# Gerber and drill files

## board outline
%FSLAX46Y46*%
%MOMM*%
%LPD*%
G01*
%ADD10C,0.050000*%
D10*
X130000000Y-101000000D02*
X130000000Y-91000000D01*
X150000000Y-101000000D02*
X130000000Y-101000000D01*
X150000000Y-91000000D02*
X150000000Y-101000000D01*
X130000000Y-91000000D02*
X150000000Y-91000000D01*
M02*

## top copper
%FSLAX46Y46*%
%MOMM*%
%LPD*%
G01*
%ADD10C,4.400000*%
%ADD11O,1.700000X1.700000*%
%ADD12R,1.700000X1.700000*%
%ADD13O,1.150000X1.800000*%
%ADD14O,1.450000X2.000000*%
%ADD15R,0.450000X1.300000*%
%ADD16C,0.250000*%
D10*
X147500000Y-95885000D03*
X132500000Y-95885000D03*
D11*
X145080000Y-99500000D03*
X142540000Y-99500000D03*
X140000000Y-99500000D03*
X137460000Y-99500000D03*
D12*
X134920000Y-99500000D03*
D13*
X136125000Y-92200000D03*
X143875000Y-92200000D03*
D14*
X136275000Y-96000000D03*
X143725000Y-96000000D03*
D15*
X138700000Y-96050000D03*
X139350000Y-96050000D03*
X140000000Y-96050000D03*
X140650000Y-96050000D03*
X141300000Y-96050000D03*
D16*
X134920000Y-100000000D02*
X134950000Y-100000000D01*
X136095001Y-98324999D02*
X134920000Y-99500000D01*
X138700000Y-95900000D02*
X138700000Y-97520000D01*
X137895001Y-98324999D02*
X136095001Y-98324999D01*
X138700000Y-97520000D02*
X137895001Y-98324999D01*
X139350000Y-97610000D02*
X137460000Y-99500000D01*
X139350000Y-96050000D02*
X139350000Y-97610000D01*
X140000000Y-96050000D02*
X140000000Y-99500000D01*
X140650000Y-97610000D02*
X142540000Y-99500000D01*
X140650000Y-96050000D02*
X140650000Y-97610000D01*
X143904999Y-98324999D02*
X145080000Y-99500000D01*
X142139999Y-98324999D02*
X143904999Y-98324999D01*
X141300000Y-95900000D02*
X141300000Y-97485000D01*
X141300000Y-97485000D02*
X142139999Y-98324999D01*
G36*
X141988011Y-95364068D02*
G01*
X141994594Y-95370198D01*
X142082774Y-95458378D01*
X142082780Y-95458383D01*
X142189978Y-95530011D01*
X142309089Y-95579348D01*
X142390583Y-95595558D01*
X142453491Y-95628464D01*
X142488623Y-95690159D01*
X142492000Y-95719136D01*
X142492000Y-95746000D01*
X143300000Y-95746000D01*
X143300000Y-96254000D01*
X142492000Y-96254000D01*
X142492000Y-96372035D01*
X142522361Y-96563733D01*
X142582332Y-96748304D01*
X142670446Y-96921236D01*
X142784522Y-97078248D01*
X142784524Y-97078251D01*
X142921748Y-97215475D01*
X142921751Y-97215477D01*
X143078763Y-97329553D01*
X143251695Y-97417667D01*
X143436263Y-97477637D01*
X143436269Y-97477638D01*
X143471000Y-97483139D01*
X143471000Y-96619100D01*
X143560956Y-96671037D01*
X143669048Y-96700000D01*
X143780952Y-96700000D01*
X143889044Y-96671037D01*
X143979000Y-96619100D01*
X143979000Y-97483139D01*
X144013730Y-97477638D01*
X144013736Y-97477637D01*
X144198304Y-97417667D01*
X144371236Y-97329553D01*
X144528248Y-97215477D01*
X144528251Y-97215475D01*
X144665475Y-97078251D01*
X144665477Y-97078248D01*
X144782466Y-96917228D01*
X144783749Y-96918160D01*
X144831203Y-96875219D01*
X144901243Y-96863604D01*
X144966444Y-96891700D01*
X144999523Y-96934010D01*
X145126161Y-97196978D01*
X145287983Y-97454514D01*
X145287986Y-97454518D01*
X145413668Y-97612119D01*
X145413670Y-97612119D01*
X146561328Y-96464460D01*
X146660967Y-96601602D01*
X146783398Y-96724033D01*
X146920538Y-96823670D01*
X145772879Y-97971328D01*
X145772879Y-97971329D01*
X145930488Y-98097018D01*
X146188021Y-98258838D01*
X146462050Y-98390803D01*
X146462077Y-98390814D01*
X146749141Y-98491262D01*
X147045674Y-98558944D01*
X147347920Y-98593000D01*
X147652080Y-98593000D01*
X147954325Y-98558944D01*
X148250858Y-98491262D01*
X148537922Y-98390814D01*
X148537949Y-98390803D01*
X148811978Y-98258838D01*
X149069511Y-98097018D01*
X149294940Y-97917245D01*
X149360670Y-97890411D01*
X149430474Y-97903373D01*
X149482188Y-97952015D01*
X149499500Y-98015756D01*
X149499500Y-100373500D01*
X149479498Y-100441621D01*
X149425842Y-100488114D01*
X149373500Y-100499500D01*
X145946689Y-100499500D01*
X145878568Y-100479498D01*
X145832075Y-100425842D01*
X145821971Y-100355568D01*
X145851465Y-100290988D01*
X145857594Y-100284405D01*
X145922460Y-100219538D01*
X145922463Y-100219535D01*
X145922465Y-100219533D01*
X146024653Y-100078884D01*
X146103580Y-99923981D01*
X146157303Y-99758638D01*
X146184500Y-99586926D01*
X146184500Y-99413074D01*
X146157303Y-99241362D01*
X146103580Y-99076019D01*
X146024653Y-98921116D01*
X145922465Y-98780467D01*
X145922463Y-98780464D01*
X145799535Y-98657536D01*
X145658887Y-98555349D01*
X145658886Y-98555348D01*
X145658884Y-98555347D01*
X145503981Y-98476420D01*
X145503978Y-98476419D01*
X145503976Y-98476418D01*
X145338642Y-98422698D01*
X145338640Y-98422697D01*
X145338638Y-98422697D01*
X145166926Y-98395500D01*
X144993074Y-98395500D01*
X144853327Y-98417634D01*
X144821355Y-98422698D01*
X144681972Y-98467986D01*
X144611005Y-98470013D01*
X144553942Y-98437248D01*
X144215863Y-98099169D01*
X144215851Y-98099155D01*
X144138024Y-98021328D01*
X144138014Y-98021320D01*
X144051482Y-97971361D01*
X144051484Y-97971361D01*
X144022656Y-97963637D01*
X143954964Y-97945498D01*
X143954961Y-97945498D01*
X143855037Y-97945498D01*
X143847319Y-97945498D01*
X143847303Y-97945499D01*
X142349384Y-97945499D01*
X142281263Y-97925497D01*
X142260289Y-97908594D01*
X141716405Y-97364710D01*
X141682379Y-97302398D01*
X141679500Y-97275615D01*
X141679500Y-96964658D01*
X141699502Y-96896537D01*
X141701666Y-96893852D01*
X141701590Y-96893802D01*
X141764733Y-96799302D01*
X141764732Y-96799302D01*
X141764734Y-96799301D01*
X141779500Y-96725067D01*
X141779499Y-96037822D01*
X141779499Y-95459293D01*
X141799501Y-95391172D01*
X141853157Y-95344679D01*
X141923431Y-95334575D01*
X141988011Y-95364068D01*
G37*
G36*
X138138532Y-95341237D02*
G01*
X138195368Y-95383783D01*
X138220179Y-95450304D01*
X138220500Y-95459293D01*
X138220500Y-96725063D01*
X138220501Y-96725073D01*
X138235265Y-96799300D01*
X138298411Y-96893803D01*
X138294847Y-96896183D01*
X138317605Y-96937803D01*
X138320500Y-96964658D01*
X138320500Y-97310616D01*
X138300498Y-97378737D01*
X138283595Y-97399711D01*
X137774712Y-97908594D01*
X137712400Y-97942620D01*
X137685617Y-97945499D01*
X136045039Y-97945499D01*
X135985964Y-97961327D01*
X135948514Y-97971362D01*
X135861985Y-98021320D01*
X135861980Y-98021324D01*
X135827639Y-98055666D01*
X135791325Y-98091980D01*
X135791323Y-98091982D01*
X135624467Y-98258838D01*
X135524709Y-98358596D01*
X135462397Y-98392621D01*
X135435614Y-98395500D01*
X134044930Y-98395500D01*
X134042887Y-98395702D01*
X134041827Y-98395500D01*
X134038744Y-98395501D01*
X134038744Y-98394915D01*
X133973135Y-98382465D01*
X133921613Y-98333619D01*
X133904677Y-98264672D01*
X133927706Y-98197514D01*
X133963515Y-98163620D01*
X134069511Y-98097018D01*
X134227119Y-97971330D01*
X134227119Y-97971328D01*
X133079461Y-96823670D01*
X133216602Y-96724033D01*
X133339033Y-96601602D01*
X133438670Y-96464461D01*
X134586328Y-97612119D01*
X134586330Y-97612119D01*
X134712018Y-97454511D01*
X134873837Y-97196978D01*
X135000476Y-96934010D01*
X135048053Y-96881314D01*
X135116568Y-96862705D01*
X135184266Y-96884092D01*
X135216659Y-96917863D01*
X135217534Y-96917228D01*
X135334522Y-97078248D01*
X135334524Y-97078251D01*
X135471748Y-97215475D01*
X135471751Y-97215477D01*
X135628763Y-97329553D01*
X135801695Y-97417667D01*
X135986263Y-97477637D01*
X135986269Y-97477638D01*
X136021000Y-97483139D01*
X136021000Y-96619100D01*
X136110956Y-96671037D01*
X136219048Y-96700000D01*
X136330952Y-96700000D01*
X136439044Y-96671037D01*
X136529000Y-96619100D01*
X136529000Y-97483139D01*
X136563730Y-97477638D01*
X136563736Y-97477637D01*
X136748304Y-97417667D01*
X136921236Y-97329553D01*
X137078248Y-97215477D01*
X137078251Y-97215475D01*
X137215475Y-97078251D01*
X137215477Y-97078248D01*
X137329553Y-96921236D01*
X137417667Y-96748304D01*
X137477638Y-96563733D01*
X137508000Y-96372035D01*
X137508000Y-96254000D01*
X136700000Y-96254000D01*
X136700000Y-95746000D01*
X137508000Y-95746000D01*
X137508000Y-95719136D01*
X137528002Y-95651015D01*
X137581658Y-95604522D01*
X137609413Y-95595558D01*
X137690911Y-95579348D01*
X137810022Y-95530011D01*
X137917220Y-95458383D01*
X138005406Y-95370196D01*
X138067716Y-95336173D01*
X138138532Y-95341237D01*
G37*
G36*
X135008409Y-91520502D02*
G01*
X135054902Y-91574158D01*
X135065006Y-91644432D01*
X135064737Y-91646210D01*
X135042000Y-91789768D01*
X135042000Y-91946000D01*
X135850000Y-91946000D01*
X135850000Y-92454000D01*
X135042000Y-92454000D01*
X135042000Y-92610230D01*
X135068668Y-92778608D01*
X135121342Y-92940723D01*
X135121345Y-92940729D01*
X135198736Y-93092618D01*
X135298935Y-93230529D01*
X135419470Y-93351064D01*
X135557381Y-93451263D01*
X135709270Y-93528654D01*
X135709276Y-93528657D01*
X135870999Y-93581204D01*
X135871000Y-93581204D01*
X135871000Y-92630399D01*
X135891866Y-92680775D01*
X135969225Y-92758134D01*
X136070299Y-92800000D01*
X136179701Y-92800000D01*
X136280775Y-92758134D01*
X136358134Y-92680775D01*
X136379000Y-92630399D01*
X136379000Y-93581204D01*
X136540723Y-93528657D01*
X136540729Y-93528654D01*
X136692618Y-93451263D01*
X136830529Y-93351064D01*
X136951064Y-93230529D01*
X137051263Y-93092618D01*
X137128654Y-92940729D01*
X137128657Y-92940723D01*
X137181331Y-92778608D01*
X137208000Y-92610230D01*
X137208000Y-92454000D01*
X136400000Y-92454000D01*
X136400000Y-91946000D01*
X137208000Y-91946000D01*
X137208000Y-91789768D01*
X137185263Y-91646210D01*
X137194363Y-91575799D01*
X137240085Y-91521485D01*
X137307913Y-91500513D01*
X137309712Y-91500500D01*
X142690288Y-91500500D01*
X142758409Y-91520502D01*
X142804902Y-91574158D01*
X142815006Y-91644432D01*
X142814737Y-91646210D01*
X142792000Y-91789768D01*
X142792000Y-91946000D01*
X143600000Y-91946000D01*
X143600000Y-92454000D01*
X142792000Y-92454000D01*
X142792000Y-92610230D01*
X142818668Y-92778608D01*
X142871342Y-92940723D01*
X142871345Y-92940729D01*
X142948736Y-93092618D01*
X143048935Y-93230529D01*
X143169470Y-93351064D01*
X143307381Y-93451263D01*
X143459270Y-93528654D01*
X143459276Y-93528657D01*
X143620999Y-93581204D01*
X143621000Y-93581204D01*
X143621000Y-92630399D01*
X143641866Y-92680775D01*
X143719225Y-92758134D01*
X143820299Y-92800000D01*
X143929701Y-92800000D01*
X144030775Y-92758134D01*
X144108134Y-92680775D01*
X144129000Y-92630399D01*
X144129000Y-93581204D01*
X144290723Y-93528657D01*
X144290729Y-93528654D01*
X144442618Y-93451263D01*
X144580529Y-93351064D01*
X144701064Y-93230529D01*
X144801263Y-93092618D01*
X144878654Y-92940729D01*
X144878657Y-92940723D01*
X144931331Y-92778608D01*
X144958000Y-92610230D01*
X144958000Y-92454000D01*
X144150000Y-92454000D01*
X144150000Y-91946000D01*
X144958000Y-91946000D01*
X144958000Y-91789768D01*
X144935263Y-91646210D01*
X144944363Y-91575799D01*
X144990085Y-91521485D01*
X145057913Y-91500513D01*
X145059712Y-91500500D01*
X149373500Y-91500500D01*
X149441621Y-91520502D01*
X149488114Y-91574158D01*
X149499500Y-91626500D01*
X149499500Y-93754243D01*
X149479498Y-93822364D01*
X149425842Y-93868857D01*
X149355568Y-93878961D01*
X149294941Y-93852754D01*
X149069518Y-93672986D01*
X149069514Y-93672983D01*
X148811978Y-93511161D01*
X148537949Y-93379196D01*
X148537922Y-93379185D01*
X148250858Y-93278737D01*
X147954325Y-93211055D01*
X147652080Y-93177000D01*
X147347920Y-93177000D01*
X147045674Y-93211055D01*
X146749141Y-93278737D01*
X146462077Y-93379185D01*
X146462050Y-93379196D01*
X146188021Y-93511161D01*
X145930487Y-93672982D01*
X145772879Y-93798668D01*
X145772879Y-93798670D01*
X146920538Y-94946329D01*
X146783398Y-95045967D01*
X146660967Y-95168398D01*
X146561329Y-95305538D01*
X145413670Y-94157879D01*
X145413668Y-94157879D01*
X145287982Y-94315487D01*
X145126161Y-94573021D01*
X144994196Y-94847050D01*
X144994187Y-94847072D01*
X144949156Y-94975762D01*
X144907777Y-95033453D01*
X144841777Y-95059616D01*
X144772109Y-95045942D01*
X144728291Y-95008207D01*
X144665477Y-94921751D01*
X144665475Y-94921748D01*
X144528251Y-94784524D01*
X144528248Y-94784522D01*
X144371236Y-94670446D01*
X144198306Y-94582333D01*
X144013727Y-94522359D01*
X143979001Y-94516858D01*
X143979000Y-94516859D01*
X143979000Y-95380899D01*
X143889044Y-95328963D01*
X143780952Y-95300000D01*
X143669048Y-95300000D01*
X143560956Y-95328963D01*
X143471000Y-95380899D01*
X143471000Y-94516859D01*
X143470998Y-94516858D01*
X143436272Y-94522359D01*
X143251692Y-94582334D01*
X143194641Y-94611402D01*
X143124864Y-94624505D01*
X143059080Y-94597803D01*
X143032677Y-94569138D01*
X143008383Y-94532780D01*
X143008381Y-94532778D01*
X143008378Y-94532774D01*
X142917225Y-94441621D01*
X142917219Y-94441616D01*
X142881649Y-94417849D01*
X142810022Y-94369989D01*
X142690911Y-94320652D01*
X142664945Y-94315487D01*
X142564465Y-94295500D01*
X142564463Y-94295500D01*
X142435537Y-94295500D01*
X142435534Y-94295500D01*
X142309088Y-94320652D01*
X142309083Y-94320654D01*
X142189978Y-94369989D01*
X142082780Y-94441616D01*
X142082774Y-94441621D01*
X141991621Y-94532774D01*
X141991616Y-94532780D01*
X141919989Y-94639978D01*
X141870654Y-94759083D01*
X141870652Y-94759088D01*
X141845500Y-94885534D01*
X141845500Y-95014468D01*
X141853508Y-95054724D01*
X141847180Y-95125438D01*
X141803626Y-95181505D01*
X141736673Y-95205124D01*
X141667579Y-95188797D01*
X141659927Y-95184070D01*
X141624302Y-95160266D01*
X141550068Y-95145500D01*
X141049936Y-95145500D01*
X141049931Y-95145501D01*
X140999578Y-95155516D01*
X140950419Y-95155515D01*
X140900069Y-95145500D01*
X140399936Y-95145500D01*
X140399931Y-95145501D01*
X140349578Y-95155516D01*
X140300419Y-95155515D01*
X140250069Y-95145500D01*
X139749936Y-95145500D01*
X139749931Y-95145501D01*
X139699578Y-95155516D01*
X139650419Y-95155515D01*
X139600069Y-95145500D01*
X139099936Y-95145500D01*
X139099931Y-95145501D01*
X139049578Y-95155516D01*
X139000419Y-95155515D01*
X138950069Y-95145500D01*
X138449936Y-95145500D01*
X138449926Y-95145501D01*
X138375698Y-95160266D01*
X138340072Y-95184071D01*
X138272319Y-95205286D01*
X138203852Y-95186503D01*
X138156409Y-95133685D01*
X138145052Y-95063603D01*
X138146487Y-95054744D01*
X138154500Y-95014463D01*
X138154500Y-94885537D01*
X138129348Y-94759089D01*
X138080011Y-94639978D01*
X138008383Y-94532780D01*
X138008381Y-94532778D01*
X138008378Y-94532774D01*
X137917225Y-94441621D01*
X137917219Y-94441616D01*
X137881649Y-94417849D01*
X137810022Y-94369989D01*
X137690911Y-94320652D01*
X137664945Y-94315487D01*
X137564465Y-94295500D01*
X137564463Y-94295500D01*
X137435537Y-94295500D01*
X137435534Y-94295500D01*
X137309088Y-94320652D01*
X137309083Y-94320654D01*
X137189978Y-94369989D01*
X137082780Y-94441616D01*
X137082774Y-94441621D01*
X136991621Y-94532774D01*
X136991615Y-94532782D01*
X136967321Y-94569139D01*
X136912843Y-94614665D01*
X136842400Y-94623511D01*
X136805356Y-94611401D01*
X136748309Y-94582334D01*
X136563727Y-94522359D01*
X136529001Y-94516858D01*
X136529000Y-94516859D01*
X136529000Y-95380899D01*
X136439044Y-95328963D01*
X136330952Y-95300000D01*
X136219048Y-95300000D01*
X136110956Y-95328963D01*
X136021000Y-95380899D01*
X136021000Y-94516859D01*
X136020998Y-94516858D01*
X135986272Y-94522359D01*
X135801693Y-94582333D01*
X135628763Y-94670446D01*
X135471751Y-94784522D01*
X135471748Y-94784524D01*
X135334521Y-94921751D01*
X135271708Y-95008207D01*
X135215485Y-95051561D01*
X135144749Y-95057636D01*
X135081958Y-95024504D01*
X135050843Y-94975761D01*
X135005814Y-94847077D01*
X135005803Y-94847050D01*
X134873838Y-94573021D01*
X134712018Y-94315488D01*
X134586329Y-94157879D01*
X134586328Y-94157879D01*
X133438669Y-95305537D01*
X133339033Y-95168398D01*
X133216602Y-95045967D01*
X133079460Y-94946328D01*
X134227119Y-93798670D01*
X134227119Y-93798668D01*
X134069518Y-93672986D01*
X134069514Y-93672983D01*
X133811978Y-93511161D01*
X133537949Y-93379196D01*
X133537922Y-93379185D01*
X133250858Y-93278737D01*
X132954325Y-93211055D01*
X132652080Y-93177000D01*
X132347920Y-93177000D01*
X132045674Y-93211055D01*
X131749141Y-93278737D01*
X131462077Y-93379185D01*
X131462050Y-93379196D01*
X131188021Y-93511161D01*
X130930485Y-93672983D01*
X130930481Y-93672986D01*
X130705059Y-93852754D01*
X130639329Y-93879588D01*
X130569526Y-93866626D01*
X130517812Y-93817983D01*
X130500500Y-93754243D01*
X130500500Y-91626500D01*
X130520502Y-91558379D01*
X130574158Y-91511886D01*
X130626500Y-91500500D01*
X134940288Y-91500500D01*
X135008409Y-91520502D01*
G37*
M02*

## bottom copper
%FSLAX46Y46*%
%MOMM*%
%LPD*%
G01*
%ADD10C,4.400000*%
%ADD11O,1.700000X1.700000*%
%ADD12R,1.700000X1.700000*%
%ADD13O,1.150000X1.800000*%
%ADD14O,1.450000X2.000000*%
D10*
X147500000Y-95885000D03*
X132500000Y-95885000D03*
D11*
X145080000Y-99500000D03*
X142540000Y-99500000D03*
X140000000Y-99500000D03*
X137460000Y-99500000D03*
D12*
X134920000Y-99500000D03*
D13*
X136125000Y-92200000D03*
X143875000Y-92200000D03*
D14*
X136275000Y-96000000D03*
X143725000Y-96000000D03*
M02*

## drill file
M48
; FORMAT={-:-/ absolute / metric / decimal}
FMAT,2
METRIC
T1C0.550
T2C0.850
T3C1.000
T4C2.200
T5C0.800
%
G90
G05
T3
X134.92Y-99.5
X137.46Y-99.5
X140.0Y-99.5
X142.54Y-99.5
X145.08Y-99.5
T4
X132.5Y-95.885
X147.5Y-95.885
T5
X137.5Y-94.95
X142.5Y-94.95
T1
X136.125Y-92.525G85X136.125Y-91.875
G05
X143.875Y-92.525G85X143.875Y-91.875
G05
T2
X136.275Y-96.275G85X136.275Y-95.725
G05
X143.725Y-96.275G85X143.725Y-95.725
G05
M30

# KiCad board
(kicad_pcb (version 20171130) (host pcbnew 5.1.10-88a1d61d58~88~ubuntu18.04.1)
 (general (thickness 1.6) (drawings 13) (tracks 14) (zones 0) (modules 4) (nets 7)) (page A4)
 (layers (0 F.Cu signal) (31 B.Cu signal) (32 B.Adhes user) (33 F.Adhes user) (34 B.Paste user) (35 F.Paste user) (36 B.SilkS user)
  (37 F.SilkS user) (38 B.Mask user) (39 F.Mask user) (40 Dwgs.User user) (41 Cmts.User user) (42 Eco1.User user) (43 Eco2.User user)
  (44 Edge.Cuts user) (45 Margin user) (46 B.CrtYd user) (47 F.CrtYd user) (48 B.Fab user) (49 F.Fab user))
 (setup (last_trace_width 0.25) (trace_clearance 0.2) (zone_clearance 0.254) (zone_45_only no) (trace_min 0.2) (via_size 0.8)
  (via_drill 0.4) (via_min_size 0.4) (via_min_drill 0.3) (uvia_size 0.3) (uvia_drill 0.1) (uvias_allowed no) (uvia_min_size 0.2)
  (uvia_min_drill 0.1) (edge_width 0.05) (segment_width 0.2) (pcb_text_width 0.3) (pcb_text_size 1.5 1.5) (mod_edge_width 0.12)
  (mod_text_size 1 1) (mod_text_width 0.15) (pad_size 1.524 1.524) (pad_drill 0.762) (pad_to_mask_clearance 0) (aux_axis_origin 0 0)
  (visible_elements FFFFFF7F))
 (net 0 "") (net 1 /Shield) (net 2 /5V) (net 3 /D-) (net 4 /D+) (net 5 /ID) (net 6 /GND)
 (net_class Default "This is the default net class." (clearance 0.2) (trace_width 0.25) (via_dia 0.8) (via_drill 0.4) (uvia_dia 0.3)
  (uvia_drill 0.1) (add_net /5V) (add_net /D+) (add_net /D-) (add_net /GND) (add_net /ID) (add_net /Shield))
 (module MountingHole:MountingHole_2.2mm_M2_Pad (layer F.Cu) (at 147.5 95.885)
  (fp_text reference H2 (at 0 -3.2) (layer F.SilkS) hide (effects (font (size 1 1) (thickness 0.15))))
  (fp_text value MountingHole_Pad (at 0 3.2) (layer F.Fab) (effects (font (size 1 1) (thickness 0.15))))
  (pad 1 thru_hole circle (at 0 0) (size 4.4 4.4) (drill 2.2) (layers *.Cu *.Mask) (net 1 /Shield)))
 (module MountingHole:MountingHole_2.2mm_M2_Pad (layer F.Cu) (at 132.5 95.885)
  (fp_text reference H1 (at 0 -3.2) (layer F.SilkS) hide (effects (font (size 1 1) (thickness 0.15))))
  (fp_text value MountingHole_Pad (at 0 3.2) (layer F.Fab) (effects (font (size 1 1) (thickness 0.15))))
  (pad 1 thru_hole circle (at 0 0) (size 4.4 4.4) (drill 2.2) (layers *.Cu *.Mask) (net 1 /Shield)))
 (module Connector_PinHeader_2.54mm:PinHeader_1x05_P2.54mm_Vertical (layer F.Cu) (at 134.92 99.5 90)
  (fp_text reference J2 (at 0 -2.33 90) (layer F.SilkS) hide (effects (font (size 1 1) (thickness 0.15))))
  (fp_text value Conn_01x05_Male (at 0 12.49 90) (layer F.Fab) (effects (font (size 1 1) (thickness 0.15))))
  (pad 5 thru_hole oval (at 0 10.16 90) (size 1.7 1.7) (drill 1) (layers *.Cu *.Mask) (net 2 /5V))
  (pad 4 thru_hole oval (at 0 7.62 90) (size 1.7 1.7) (drill 1) (layers *.Cu *.Mask) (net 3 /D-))
  (pad 3 thru_hole oval (at 0 5.08 90) (size 1.7 1.7) (drill 1) (layers *.Cu *.Mask) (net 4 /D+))
  (pad 2 thru_hole oval (at 0 2.54 90) (size 1.7 1.7) (drill 1) (layers *.Cu *.Mask) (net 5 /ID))
  (pad 1 thru_hole rect (at 0 0 90) (size 1.7 1.7) (drill 1) (layers *.Cu *.Mask) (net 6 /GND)))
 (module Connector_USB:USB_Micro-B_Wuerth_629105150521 (layer F.Cu) (at 140 94.15 180)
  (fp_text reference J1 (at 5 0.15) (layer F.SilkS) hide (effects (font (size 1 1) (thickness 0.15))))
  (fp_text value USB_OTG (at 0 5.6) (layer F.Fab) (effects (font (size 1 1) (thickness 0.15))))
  (pad "" np_thru_hole oval (at 2.5 -0.8 180) (size 0.8 0.8) (drill 0.8) (layers *.Cu *.Mask))
  (pad "" np_thru_hole oval (at -2.5 -0.8 180) (size 0.8 0.8) (drill 0.8) (layers *.Cu *.Mask))
  (pad 6 thru_hole oval (at 3.875 1.95 180) (size 1.15 1.8) (drill oval 0.55 1.2) (layers *.Cu *.Mask) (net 1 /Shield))
  (pad 6 thru_hole oval (at -3.875 1.95 180) (size 1.15 1.8) (drill oval 0.55 1.2) (layers *.Cu *.Mask) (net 1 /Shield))
  (pad 6 thru_hole oval (at 3.725 -1.85 180) (size 1.45 2) (drill oval 0.85 1.4) (layers *.Cu *.Mask) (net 1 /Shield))
  (pad 6 thru_hole oval (at -3.725 -1.85 180) (size 1.45 2) (drill oval 0.85 1.4) (layers *.Cu *.Mask) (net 1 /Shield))
  (pad 5 smd rect (at 1.3 -1.9 180) (size 0.45 1.3) (layers F.Cu F.Paste F.Mask) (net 6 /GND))
  (pad 4 smd rect (at 0.65 -1.9 180) (size 0.45 1.3) (layers F.Cu F.Paste F.Mask) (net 5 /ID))
  (pad 3 smd rect (at 0 -1.9 180) (size 0.45 1.3) (layers F.Cu F.Paste F.Mask) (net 4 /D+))
  (pad 2 smd rect (at -0.65 -1.9 180) (size 0.45 1.3) (layers F.Cu F.Paste F.Mask) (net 3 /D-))
  (pad 1 smd rect (at -1.3 -1.9 180) (size 0.45 1.3) (layers F.Cu F.Paste F.Mask) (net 2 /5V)))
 (gr_line (start 130 101) (end 130 91) (layer Edge.Cuts) (width 0.05))
 (gr_line (start 150 101) (end 130 101) (layer Edge.Cuts) (width 0.05))
 (gr_line (start 150 91) (end 150 101) (layer Edge.Cuts) (width 0.05))
 (gr_line (start 130 91) (end 150 91) (layer Edge.Cuts) (width 0.05))
 (segment (start 134.92 100) (end 134.95 100) (width 0.25) (layer F.Cu) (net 6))
 (segment (start 136.095001 98.324999) (end 134.92 99.5) (width 0.25) (layer F.Cu) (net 6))
 (segment (start 138.7 95.9) (end 138.7 97.52) (width 0.25) (layer F.Cu) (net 6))
 (segment (start 137.895001 98.324999) (end 136.095001 98.324999) (width 0.25) (layer F.Cu) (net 6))
 (segment (start 138.7 97.52) (end 137.895001 98.324999) (width 0.25) (layer F.Cu) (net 6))
 (segment (start 139.35 97.61) (end 137.46 99.5) (width 0.25) (layer F.Cu) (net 5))
 (segment (start 139.35 96.05) (end 139.35 97.61) (width 0.25) (layer F.Cu) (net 5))
 (segment (start 140 96.05) (end 140 99.5) (width 0.25) (layer F.Cu) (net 4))
 (segment (start 140.65 97.61) (end 142.54 99.5) (width 0.25) (layer F.Cu) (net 3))
 (segment (start 140.65 96.05) (end 140.65 97.61) (width 0.25) (layer F.Cu) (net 3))
 (segment (start 143.904999 98.324999) (end 145.08 99.5) (width 0.25) (layer F.Cu) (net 2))
 (segment (start 142.139999 98.324999) (end 143.904999 98.324999) (width 0.25) (layer F.Cu) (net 2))
 (segment (start 141.3 95.9) (end 141.3 97.485) (width 0.25) (layer F.Cu) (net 2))
 (segment (start 141.3 97.485) (end 142.139999 98.324999) (width 0.25) (layer F.Cu) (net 2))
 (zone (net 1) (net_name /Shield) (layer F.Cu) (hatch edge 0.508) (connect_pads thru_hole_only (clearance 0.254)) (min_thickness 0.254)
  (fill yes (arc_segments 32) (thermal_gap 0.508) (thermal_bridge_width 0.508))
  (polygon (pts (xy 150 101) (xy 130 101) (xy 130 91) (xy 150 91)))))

